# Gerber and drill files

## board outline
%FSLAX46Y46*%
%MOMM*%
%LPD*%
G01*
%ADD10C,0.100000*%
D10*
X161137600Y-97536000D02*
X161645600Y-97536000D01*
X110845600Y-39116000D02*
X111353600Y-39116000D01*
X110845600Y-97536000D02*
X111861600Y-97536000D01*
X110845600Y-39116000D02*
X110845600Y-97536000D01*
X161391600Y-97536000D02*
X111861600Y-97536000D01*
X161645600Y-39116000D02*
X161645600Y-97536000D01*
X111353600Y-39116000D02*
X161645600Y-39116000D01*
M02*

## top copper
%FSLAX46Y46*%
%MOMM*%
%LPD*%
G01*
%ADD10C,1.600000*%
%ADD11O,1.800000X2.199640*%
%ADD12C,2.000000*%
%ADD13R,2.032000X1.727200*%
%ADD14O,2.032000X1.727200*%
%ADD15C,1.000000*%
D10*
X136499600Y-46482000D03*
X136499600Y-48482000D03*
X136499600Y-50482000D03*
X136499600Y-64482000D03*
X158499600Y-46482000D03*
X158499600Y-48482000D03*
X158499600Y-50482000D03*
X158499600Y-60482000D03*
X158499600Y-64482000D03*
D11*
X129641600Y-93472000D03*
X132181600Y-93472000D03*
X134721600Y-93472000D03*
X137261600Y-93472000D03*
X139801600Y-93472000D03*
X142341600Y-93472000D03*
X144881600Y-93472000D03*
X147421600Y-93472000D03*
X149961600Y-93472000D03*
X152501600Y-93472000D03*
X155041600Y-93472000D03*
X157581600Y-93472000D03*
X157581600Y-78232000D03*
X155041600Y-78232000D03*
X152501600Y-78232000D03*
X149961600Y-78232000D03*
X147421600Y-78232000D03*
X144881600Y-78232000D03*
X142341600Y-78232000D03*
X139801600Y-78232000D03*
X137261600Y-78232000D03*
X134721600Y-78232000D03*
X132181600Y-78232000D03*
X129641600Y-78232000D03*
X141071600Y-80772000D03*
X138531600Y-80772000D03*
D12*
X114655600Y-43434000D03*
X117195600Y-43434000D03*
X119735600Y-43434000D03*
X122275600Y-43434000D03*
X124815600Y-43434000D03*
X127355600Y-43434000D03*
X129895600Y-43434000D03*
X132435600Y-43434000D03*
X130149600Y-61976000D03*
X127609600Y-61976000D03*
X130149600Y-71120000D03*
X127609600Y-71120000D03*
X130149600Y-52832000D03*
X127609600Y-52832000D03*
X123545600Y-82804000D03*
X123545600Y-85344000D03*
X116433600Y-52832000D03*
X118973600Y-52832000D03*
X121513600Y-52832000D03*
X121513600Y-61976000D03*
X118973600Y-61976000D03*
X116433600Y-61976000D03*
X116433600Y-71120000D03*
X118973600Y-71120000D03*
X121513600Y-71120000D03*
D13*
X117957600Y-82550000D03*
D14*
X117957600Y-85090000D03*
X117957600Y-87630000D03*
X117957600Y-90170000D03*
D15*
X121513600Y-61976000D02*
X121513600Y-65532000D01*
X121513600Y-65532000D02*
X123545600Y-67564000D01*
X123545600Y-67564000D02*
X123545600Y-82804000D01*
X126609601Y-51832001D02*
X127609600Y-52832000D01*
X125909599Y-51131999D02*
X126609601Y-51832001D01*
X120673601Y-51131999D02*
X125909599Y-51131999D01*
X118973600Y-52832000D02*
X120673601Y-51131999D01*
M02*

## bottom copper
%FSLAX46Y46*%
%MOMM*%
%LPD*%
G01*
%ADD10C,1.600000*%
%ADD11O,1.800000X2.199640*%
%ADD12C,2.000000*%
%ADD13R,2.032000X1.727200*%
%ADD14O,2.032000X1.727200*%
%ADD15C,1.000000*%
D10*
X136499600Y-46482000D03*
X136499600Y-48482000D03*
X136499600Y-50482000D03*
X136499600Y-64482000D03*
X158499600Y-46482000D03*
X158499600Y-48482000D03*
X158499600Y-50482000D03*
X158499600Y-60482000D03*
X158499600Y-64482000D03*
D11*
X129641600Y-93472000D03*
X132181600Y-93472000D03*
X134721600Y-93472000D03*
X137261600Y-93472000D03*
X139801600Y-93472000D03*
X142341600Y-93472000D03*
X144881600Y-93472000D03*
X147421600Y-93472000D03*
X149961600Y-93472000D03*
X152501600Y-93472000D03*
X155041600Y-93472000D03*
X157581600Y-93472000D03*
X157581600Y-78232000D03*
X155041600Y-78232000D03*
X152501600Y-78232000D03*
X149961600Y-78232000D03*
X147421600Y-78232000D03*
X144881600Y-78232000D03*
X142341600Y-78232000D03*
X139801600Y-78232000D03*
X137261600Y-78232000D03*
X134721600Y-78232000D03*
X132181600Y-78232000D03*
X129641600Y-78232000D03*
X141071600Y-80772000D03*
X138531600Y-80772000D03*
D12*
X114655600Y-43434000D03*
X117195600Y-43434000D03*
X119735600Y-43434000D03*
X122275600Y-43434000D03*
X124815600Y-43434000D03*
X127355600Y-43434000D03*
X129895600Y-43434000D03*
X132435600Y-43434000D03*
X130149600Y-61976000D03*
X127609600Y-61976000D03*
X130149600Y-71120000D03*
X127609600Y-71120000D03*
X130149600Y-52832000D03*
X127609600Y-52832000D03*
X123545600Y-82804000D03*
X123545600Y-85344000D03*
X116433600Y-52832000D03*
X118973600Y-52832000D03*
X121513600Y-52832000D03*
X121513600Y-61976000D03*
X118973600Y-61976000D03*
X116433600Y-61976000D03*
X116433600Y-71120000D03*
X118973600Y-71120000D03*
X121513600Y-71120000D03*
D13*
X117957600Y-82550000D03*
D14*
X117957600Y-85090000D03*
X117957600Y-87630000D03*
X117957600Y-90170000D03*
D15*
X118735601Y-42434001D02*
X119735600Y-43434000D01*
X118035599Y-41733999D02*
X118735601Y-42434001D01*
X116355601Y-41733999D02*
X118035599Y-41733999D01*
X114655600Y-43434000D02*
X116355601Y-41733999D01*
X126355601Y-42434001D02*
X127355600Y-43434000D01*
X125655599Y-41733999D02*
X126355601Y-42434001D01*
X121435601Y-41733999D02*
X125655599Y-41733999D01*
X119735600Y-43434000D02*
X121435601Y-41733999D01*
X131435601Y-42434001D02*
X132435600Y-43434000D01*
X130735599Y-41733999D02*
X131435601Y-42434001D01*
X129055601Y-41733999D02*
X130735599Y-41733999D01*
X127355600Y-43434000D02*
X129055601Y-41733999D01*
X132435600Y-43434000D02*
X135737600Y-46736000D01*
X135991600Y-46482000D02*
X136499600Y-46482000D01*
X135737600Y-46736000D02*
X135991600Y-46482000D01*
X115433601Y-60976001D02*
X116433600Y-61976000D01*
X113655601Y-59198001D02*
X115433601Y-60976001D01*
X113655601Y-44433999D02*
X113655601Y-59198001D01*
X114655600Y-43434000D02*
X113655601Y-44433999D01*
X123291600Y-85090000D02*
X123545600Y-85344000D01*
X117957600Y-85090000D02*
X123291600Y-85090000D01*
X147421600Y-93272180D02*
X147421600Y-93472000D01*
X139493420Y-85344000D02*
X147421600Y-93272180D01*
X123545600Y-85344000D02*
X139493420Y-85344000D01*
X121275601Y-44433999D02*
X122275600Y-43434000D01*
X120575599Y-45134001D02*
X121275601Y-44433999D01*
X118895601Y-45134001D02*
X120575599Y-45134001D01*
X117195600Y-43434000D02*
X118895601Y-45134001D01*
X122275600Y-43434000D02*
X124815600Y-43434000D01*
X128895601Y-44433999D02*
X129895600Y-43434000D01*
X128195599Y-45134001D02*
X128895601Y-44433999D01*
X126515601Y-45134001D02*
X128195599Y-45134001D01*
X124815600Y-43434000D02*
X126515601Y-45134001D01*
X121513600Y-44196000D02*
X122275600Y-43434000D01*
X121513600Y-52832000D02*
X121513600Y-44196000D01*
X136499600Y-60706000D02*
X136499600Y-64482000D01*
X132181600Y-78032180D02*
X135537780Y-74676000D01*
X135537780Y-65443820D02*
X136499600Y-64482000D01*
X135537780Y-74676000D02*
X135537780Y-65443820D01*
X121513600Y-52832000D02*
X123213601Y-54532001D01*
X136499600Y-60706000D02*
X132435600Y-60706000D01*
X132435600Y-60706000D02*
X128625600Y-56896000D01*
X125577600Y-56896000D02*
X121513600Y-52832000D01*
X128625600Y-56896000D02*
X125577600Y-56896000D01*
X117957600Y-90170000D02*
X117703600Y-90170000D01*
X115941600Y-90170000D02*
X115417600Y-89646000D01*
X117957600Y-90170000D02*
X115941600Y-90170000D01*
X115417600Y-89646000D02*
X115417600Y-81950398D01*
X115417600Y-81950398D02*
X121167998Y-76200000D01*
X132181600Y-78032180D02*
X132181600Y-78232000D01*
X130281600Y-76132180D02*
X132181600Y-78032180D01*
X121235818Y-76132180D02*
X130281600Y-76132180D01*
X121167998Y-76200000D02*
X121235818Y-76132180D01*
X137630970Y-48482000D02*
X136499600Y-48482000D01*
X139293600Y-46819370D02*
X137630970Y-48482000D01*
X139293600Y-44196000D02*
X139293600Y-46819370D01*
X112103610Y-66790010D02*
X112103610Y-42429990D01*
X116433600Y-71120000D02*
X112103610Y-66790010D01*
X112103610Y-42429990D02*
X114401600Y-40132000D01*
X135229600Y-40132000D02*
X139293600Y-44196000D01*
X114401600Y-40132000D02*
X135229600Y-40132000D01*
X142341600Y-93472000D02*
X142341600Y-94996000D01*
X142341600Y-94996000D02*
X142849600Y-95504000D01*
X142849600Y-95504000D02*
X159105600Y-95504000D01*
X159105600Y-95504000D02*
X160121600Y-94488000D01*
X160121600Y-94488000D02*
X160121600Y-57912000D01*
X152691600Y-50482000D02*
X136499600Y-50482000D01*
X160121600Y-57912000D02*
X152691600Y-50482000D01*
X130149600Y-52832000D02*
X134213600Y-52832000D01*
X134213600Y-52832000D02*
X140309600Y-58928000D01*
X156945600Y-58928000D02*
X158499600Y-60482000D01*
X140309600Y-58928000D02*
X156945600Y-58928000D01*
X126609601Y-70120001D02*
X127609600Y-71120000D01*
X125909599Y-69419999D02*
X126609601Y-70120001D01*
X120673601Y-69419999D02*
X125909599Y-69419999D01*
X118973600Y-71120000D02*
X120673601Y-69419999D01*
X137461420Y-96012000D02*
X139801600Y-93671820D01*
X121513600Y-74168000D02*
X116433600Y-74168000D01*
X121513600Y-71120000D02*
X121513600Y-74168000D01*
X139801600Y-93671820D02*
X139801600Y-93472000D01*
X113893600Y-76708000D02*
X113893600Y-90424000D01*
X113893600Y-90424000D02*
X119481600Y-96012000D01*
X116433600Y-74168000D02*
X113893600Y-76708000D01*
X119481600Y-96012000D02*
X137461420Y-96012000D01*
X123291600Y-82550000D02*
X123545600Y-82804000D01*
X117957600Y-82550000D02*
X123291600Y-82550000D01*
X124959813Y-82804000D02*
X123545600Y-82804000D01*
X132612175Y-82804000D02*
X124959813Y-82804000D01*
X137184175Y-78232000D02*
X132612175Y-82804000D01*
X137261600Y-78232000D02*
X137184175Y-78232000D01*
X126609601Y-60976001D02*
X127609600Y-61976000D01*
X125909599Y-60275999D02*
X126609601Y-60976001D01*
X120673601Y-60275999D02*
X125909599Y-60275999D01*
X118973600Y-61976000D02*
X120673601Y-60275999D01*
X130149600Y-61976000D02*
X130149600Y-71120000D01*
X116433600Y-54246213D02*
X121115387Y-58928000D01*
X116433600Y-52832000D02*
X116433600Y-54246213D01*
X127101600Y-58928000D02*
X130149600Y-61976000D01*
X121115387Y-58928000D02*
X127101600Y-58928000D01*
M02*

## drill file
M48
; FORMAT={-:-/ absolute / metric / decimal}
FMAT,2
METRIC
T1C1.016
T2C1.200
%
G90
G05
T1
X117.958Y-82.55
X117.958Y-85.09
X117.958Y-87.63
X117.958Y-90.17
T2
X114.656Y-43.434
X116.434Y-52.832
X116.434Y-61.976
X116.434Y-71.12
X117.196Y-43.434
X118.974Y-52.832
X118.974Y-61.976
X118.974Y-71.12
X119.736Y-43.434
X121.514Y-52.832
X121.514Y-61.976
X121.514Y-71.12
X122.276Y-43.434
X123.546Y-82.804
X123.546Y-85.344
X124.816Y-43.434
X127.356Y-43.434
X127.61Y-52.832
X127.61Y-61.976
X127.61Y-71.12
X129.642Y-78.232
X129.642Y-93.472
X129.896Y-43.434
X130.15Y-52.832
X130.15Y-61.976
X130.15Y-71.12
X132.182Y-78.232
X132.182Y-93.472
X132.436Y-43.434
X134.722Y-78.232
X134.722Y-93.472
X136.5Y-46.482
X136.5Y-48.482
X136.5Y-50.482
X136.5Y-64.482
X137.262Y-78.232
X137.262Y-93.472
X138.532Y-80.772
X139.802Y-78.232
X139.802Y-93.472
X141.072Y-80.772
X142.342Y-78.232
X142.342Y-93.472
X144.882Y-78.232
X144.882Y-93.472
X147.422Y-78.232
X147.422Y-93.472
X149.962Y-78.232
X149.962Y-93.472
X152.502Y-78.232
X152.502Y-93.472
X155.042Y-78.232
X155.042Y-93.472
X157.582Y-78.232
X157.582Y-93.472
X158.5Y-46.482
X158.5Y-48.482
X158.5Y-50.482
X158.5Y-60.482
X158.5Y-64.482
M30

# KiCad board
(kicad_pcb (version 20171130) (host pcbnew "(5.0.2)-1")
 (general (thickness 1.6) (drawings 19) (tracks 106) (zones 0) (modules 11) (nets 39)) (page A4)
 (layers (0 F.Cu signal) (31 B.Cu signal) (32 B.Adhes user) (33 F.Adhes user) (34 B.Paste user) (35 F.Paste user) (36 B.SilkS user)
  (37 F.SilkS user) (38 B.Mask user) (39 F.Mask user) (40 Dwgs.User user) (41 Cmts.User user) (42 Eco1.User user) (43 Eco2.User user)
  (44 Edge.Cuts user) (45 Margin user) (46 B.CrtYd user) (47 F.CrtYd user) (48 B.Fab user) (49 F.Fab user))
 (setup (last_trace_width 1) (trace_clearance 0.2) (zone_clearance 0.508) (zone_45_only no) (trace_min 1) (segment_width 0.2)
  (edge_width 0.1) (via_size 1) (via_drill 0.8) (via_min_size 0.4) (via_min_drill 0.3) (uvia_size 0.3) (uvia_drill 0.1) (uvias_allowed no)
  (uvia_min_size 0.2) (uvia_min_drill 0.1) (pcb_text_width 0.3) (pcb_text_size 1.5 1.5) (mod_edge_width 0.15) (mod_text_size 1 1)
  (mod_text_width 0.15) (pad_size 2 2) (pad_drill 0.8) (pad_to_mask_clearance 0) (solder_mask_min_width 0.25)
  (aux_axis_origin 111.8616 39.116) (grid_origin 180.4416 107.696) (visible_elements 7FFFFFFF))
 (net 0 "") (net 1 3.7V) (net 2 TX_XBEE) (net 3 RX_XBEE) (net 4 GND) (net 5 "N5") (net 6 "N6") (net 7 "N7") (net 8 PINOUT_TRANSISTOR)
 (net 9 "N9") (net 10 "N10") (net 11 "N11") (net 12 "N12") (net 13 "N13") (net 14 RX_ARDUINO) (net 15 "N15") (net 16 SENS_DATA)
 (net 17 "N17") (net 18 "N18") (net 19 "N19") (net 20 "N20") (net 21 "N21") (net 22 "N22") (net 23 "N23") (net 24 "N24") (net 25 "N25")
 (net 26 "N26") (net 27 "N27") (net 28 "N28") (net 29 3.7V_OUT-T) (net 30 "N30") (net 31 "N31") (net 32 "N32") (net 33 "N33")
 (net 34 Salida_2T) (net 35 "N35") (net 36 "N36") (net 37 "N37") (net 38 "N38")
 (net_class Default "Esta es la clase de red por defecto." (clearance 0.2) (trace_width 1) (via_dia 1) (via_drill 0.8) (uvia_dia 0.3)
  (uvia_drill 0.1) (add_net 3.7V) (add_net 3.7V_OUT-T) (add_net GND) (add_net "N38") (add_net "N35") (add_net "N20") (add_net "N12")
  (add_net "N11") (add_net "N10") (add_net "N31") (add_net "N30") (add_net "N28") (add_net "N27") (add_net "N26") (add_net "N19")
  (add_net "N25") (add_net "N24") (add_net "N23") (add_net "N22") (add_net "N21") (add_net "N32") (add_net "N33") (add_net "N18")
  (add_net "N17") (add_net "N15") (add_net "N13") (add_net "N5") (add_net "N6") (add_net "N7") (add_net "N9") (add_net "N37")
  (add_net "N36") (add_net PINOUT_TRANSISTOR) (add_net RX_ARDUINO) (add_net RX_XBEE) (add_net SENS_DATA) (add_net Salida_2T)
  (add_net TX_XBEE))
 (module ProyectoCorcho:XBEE (layer F.Cu) (at 135.2296 45.212)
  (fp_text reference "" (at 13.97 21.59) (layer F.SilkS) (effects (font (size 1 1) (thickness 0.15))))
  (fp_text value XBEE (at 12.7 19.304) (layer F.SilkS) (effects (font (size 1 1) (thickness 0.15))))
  (pad 1 thru_hole circle (at 1.27 1.27) (size 1.6 1.6) (drill 1.2) (layers *.Cu *.Mask) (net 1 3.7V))
  (pad 2 thru_hole circle (at 1.27 3.27) (size 1.6 1.6) (drill 1.2) (layers *.Cu *.Mask) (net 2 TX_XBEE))
  (pad 3 thru_hole circle (at 1.27 5.27) (size 1.6 1.6) (drill 1.2) (layers *.Cu *.Mask) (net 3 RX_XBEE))
  (pad 4 thru_hole circle (at 1.27 19.27) (size 1.6 1.6) (drill 1.2) (layers *.Cu *.Mask) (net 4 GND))
  (pad 5 thru_hole circle (at 23.27 1.27) (size 1.6 1.6) (drill 1.2) (layers *.Cu *.Mask) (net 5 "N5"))
  (pad 6 thru_hole circle (at 23.27 3.27) (size 1.6 1.6) (drill 1.2) (layers *.Cu *.Mask) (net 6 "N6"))
  (pad 7 thru_hole circle (at 23.27 5.27) (size 1.6 1.6) (drill 1.2) (layers *.Cu *.Mask) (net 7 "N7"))
  (pad 8 thru_hole circle (at 23.27 15.27) (size 1.6 1.6) (drill 1.2) (layers *.Cu *.Mask) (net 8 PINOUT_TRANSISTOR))
  (pad 9 thru_hole circle (at 23.27 19.27) (size 1.6 1.6) (drill 1.2) (layers *.Cu *.Mask) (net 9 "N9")))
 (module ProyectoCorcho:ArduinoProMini (layer F.Cu) (at 143.6116 85.852)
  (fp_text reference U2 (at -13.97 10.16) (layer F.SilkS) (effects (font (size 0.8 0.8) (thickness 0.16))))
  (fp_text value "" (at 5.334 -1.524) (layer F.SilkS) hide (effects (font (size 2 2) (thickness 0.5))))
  (pad 12 thru_hole oval (at -13.97 7.62) (size 1.8 2.19964) (drill 1.2) (layers *.Cu *.Mask) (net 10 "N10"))
  (pad 11 thru_hole oval (at -11.43 7.62) (size 1.8 2.19964) (drill 1.2) (layers *.Cu *.Mask) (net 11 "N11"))
  (pad 10 thru_hole oval (at -8.89 7.62) (size 1.8 2.19964) (drill 1.2) (layers *.Cu *.Mask) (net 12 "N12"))
  (pad 9 thru_hole oval (at -6.35 7.62) (size 1.8 2.19964) (drill 1.2) (layers *.Cu *.Mask) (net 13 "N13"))
  (pad 8 thru_hole oval (at -3.81 7.62) (size 1.8 2.19964) (drill 1.2) (layers *.Cu *.Mask) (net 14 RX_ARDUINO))
  (pad 7 thru_hole oval (at -1.27 7.62) (size 1.8 2.19964) (drill 1.2) (layers *.Cu *.Mask) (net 3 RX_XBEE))
  (pad 6 thru_hole oval (at 1.27 7.62) (size 1.8 2.19964) (drill 1.2) (layers *.Cu *.Mask) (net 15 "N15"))
  (pad 5 thru_hole oval (at 3.81 7.62) (size 1.8 2.19964) (drill 1.2) (layers *.Cu *.Mask) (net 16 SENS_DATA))
  (pad 4 thru_hole oval (at 6.35 7.62) (size 1.8 2.19964) (drill 1.2) (layers *.Cu *.Mask) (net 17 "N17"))
  (pad 3 thru_hole oval (at 8.89 7.62) (size 1.8 2.19964) (drill 1.2) (layers *.Cu *.Mask) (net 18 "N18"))
  (pad 2 thru_hole oval (at 11.43 7.62) (size 1.8 2.19964) (drill 1.2) (layers *.Cu *.Mask) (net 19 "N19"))
  (pad 1 thru_hole oval (at 13.97 7.62) (size 1.8 2.19964) (drill 1.2) (layers *.Cu *.Mask) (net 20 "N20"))
  (pad 24 thru_hole oval (at 13.97 -7.62) (size 1.8 2.19964) (drill 1.2) (layers *.Cu *.Mask) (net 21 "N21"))
  (pad 23 thru_hole oval (at 11.43 -7.62) (size 1.8 2.19964) (drill 1.2) (layers *.Cu *.Mask) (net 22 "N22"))
  (pad 22 thru_hole oval (at 8.89 -7.62) (size 1.8 2.19964) (drill 1.2) (layers *.Cu *.Mask) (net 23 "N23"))
  (pad 21 thru_hole oval (at 6.35 -7.62) (size 1.8 2.19964) (drill 1.2) (layers *.Cu *.Mask) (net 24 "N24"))
  (pad 20 thru_hole oval (at 3.81 -7.62) (size 1.8 2.19964) (drill 1.2) (layers *.Cu *.Mask) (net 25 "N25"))
  (pad 19 thru_hole oval (at 1.27 -7.62) (size 1.8 2.19964) (drill 1.2) (layers *.Cu *.Mask) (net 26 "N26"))
  (pad 18 thru_hole oval (at -1.27 -7.62) (size 1.8 2.19964) (drill 1.2) (layers *.Cu *.Mask) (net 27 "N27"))
  (pad 17 thru_hole oval (at -3.81 -7.62) (size 1.8 2.19964) (drill 1.2) (layers *.Cu *.Mask) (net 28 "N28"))
  (pad 16 thru_hole oval (at -6.35 -7.62) (size 1.8 2.19964) (drill 1.2) (layers *.Cu *.Mask) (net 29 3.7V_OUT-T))
  (pad 15 thru_hole oval (at -8.89 -7.62) (size 1.8 2.19964) (drill 1.2) (layers *.Cu *.Mask) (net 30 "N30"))
  (pad 14 thru_hole oval (at -11.43 -7.62) (size 1.8 2.19964) (drill 1.2) (layers *.Cu *.Mask) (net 4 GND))
  (pad 13 thru_hole oval (at -13.97 -7.62) (size 1.8 2.19964) (drill 1.2) (layers *.Cu *.Mask) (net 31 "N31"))
  (pad 25 thru_hole oval (at -2.54 -5.08) (size 1.8 2.19964) (drill 1.2) (layers *.Cu *.Mask) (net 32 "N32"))
  (pad 26 thru_hole oval (at -5.08 -5.08) (size 1.8 2.19964) (drill 1.2) (layers *.Cu *.Mask) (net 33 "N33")))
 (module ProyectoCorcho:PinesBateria (layer F.Cu) (at 113.3856 42.164)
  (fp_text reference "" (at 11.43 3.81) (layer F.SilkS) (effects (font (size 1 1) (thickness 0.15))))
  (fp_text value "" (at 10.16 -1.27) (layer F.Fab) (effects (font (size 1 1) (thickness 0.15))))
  (pad 1 thru_hole circle (at 1.27 1.27) (size 2 2) (drill 1.2) (layers *.Cu *.Mask) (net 1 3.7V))
  (pad 2 thru_hole circle (at 3.81 1.27) (size 2 2) (drill 1.2) (layers *.Cu *.Mask) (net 4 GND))
  (pad 3 thru_hole circle (at 6.35 1.27) (size 2 2) (drill 1.2) (layers *.Cu *.Mask) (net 1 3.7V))
  (pad 4 thru_hole circle (at 8.89 1.27) (size 2 2) (drill 1.2) (layers *.Cu *.Mask) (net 4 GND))
  (pad 5 thru_hole circle (at 11.43 1.27) (size 2 2) (drill 1.2) (layers *.Cu *.Mask) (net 4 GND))
  (pad 6 thru_hole circle (at 13.97 1.27) (size 2 2) (drill 1.2) (layers *.Cu *.Mask) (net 1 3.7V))
  (pad 7 thru_hole circle (at 16.51 1.27) (size 2 2) (drill 1.2) (layers *.Cu *.Mask) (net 4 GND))
  (pad 8 thru_hole circle (at 19.05 1.27) (size 2 2) (drill 1.2) (layers *.Cu *.Mask) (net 1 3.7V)))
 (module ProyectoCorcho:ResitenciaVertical (layer F.Cu) (at 127.6096 61.976)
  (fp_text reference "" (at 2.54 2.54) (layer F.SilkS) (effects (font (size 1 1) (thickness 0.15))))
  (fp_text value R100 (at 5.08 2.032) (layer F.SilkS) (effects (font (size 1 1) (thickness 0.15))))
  (pad 2 thru_hole circle (at 2.54 0) (size 2 2) (drill 1.2) (layers *.Cu *.Mask) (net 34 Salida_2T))
  (pad 1 thru_hole circle (at 0 0) (size 2 2) (drill 1.2) (layers *.Cu *.Mask) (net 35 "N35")))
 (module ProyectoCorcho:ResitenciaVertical (layer F.Cu) (at 127.6096 71.12)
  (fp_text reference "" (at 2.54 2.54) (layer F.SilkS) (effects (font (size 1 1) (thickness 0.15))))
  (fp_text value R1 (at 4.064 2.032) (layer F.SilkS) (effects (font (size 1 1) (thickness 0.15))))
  (pad 2 thru_hole circle (at 2.54 0) (size 2 2) (drill 1.2) (layers *.Cu *.Mask) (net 34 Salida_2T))
  (pad 1 thru_hole circle (at 0 0) (size 2 2) (drill 1.2) (layers *.Cu *.Mask) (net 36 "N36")))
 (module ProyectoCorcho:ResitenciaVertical (layer F.Cu) (at 127.6096 52.832)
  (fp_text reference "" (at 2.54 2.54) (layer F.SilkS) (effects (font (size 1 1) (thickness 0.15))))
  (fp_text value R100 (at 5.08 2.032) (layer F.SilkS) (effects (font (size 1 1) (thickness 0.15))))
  (pad 2 thru_hole circle (at 2.54 0) (size 2 2) (drill 1.2) (layers *.Cu *.Mask) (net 8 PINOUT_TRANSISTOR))
  (pad 1 thru_hole circle (at 0 0) (size 2 2) (drill 1.2) (layers *.Cu *.Mask) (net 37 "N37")))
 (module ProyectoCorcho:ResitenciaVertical (layer F.Cu) (at 123.5456 82.804 270)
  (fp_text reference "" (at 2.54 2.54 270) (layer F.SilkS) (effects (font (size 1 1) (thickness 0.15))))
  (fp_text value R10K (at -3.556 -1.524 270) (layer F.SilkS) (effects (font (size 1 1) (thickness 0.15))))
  (pad 1 thru_hole circle (at 0 0 270) (size 2 2) (drill 1.2) (layers *.Cu *.Mask) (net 29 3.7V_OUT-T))
  (pad 2 thru_hole circle (at 2.54 0 270) (size 2 2) (drill 1.2) (layers *.Cu *.Mask) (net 16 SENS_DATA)))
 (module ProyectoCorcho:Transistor (layer F.Cu) (at 118.9736 52.832)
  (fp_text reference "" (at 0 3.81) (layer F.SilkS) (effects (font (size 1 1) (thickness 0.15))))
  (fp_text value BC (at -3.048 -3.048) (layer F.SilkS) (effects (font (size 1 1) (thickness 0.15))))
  (pad 1 thru_hole circle (at -2.54 0) (size 2 2) (drill 1.2) (layers *.Cu *.Mask) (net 34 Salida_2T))
  (pad 2 thru_hole circle (at 0 0) (size 2 2) (drill 1.2) (layers *.Cu *.Mask) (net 37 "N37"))
  (pad 3 thru_hole circle (at 2.54 0) (size 2 2) (drill 1.2) (layers *.Cu *.Mask) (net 4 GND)))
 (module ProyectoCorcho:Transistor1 (layer B.Cu) (at 118.9736 61.976)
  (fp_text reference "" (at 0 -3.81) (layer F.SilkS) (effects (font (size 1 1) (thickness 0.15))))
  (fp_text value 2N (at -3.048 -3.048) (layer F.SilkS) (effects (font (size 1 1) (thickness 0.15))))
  (pad 3 thru_hole circle (at 2.54 0) (size 2 2) (drill 1.2) (layers *.Cu *.Mask) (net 29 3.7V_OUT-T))
  (pad 2 thru_hole circle (at 0 0) (size 2 2) (drill 1.2) (layers *.Cu *.Mask) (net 35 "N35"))
  (pad 1 thru_hole circle (at -2.54 0) (size 2 2) (drill 1.2) (layers *.Cu *.Mask) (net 1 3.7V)))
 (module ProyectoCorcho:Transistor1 (layer F.Cu) (at 118.9736 71.12)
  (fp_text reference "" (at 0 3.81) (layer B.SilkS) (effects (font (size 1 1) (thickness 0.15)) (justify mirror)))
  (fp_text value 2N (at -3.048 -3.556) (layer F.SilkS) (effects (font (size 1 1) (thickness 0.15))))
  (pad 1 thru_hole circle (at -2.54 0) (size 2 2) (drill 1.2) (layers *.Cu *.Mask) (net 2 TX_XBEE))
  (pad 2 thru_hole circle (at 0 0) (size 2 2) (drill 1.2) (layers *.Cu *.Mask) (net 36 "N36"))
  (pad 3 thru_hole circle (at 2.54 0) (size 2 2) (drill 1.2) (layers *.Cu *.Mask) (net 14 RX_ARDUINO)))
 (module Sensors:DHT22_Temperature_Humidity (layer F.Cu) (at 117.9576 86.36 270)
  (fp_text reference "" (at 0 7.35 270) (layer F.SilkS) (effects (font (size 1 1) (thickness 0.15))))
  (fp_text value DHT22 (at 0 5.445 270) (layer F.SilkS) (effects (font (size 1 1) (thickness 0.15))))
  (pad 1 thru_hole rect (at -3.81 0) (size 2.032 1.7272) (drill 1.016) (layers *.Cu *.Mask F.SilkS) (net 29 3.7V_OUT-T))
  (pad 2 thru_hole oval (at -1.27 0) (size 2.032 1.7272) (drill 1.016) (layers *.Cu *.Mask F.SilkS) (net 16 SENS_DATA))
  (pad 3 thru_hole oval (at 1.27 0) (size 2.032 1.7272) (drill 1.016) (layers *.Cu *.Mask F.SilkS) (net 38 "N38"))
  (pad 4 thru_hole oval (at 3.81 0) (size 2.032 1.7272) (drill 1.016) (layers *.Cu *.Mask F.SilkS) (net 4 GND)))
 (gr_line (start 161.1376 97.536) (end 161.6456 97.536) (layer Edge.Cuts) (width 0.1))
 (gr_line (start 110.8456 39.116) (end 111.3536 39.116) (layer Edge.Cuts) (width 0.1))
 (gr_line (start 110.8456 97.536) (end 111.8616 97.536) (layer Edge.Cuts) (width 0.1))
 (gr_line (start 110.8456 39.116) (end 110.8456 97.536) (layer Edge.Cuts) (width 0.1))
 (gr_line (start 161.3916 97.536) (end 111.8616 97.536) (layer Edge.Cuts) (width 0.1))
 (gr_line (start 161.6456 39.116) (end 161.6456 97.536) (layer Edge.Cuts) (width 0.1))
 (gr_line (start 111.3536 39.116) (end 161.6456 39.116) (layer Edge.Cuts) (width 0.1))
 (segment (start 118.735601 42.434001) (end 119.7356 43.434) (width 1) (layer B.Cu) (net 1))
 (segment (start 118.035599 41.733999) (end 118.735601 42.434001) (width 1) (layer B.Cu) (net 1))
 (segment (start 116.355601 41.733999) (end 118.035599 41.733999) (width 1) (layer B.Cu) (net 1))
 (segment (start 114.6556 43.434) (end 116.355601 41.733999) (width 1) (layer B.Cu) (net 1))
 (segment (start 126.355601 42.434001) (end 127.3556 43.434) (width 1) (layer B.Cu) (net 1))
 (segment (start 125.655599 41.733999) (end 126.355601 42.434001) (width 1) (layer B.Cu) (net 1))
 (segment (start 121.435601 41.733999) (end 125.655599 41.733999) (width 1) (layer B.Cu) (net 1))
 (segment (start 119.7356 43.434) (end 121.435601 41.733999) (width 1) (layer B.Cu) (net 1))
 (segment (start 131.435601 42.434001) (end 132.4356 43.434) (width 1) (layer B.Cu) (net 1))
 (segment (start 130.735599 41.733999) (end 131.435601 42.434001) (width 1) (layer B.Cu) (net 1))
 (segment (start 129.055601 41.733999) (end 130.735599 41.733999) (width 1) (layer B.Cu) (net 1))
 (segment (start 127.3556 43.434) (end 129.055601 41.733999) (width 1) (layer B.Cu) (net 1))
 (segment (start 132.4356 43.434) (end 135.7376 46.736) (width 1) (layer B.Cu) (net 1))
 (segment (start 135.9916 46.482) (end 136.4996 46.482) (width 1) (layer B.Cu) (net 1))
 (segment (start 135.7376 46.736) (end 135.9916 46.482) (width 1) (layer B.Cu) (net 1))
 (segment (start 115.433601 60.976001) (end 116.4336 61.976) (width 1) (layer B.Cu) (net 1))
 (segment (start 113.655601 59.198001) (end 115.433601 60.976001) (width 1) (layer B.Cu) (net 1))
 (segment (start 113.655601 44.433999) (end 113.655601 59.198001) (width 1) (layer B.Cu) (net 1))
 (segment (start 114.6556 43.434) (end 113.655601 44.433999) (width 1) (layer B.Cu) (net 1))
 (segment (start 123.2916 85.09) (end 123.5456 85.344) (width 1) (layer B.Cu) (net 16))
 (segment (start 117.9576 85.09) (end 123.2916 85.09) (width 1) (layer B.Cu) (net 16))
 (segment (start 147.4216 93.27218) (end 147.4216 93.472) (width 1) (layer B.Cu) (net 16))
 (segment (start 139.49342 85.344) (end 147.4216 93.27218) (width 1) (layer B.Cu) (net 16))
 (segment (start 123.5456 85.344) (end 139.49342 85.344) (width 1) (layer B.Cu) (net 16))
 (segment (start 121.275601 44.433999) (end 122.2756 43.434) (width 1) (layer B.Cu) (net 4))
 (segment (start 120.575599 45.134001) (end 121.275601 44.433999) (width 1) (layer B.Cu) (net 4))
 (segment (start 118.895601 45.134001) (end 120.575599 45.134001) (width 1) (layer B.Cu) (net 4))
 (segment (start 117.1956 43.434) (end 118.895601 45.134001) (width 1) (layer B.Cu) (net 4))
 (segment (start 122.2756 43.434) (end 124.8156 43.434) (width 1) (layer B.Cu) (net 4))
 (segment (start 128.895601 44.433999) (end 129.8956 43.434) (width 1) (layer B.Cu) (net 4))
 (segment (start 128.195599 45.134001) (end 128.895601 44.433999) (width 1) (layer B.Cu) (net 4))
 (segment (start 126.515601 45.134001) (end 128.195599 45.134001) (width 1) (layer B.Cu) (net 4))
 (segment (start 124.8156 43.434) (end 126.515601 45.134001) (width 1) (layer B.Cu) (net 4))
 (segment (start 121.5136 44.196) (end 122.2756 43.434) (width 1) (layer B.Cu) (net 4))
 (segment (start 121.5136 52.832) (end 121.5136 44.196) (width 1) (layer B.Cu) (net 4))
 (segment (start 136.4996 60.706) (end 136.4996 64.482) (width 1) (layer B.Cu) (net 4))
 (segment (start 132.1816 78.03218) (end 135.53778 74.676) (width 1) (layer B.Cu) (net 4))
 (segment (start 135.53778 65.44382) (end 136.4996 64.482) (width 1) (layer B.Cu) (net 4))
 (segment (start 135.53778 74.676) (end 135.53778 65.44382) (width 1) (layer B.Cu) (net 4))
 (segment (start 121.5136 52.832) (end 123.213601 54.532001) (width 1) (layer B.Cu) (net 4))
 (segment (start 136.4996 60.706) (end 132.4356 60.706) (width 1) (layer B.Cu) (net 4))
 (segment (start 132.4356 60.706) (end 128.6256 56.896) (width 1) (layer B.Cu) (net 4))
 (segment (start 125.5776 56.896) (end 121.5136 52.832) (width 1) (layer B.Cu) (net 4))
 (segment (start 128.6256 56.896) (end 125.5776 56.896) (width 1) (layer B.Cu) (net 4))
 (segment (start 117.9576 90.17) (end 117.7036 90.17) (width 1) (layer B.Cu) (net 4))
 (segment (start 115.9416 90.17) (end 115.4176 89.646) (width 1) (layer B.Cu) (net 4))
 (segment (start 117.9576 90.17) (end 115.9416 90.17) (width 1) (layer B.Cu) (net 4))
 (segment (start 115.4176 89.646) (end 115.4176 81.950398) (width 1) (layer B.Cu) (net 4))
 (segment (start 115.4176 81.950398) (end 121.167998 76.2) (width 1) (layer B.Cu) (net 4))
 (segment (start 132.1816 78.03218) (end 132.1816 78.232) (width 1) (layer B.Cu) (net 4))
 (segment (start 130.2816 76.13218) (end 132.1816 78.03218) (width 1) (layer B.Cu) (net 4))
 (segment (start 121.235818 76.13218) (end 130.2816 76.13218) (width 1) (layer B.Cu) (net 4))
 (segment (start 121.167998 76.2) (end 121.235818 76.13218) (width 1) (layer B.Cu) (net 4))
 (segment (start 137.63097 48.482) (end 136.4996 48.482) (width 1) (layer B.Cu) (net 2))
 (segment (start 139.2936 46.81937) (end 137.63097 48.482) (width 1) (layer B.Cu) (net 2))
 (segment (start 139.2936 44.196) (end 139.2936 46.81937) (width 1) (layer B.Cu) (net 2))
 (segment (start 112.10361 66.79001) (end 112.10361 42.42999) (width 1) (layer B.Cu) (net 2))
 (segment (start 116.4336 71.12) (end 112.10361 66.79001) (width 1) (layer B.Cu) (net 2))
 (segment (start 112.10361 42.42999) (end 114.4016 40.132) (width 1) (layer B.Cu) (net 2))
 (segment (start 135.2296 40.132) (end 139.2936 44.196) (width 1) (layer B.Cu) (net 2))
 (segment (start 114.4016 40.132) (end 135.2296 40.132) (width 1) (layer B.Cu) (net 2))
 (segment (start 142.3416 93.472) (end 142.3416 94.996) (width 1) (layer B.Cu) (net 3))
 (segment (start 142.3416 94.996) (end 142.8496 95.504) (width 1) (layer B.Cu) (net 3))
 (segment (start 142.8496 95.504) (end 159.1056 95.504) (width 1) (layer B.Cu) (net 3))
 (segment (start 159.1056 95.504) (end 160.1216 94.488) (width 1) (layer B.Cu) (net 3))
 (segment (start 160.1216 94.488) (end 160.1216 57.912) (width 1) (layer B.Cu) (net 3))
 (segment (start 152.6916 50.482) (end 136.4996 50.482) (width 1) (layer B.Cu) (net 3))
 (segment (start 160.1216 57.912) (end 152.6916 50.482) (width 1) (layer B.Cu) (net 3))
 (segment (start 130.1496 52.832) (end 134.2136 52.832) (width 1) (layer B.Cu) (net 8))
 (segment (start 134.2136 52.832) (end 140.3096 58.928) (width 1) (layer B.Cu) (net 8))
 (segment (start 156.9456 58.928) (end 158.4996 60.482) (width 1) (layer B.Cu) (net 8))
 (segment (start 140.3096 58.928) (end 156.9456 58.928) (width 1) (layer B.Cu) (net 8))
 (segment (start 126.609601 70.120001) (end 127.6096 71.12) (width 1) (layer B.Cu) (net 36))
 (segment (start 125.909599 69.419999) (end 126.609601 70.120001) (width 1) (layer B.Cu) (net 36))
 (segment (start 120.673601 69.419999) (end 125.909599 69.419999) (width 1) (layer B.Cu) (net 36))
 (segment (start 118.9736 71.12) (end 120.673601 69.419999) (width 1) (layer B.Cu) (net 36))
 (segment (start 137.46142 96.012) (end 139.8016 93.67182) (width 1) (layer B.Cu) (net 14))
 (segment (start 121.5136 74.168) (end 116.4336 74.168) (width 1) (layer B.Cu) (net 14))
 (segment (start 121.5136 71.12) (end 121.5136 74.168) (width 1) (layer B.Cu) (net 14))
 (segment (start 139.8016 93.67182) (end 139.8016 93.472) (width 1) (layer B.Cu) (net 14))
 (segment (start 113.8936 76.708) (end 113.8936 90.424) (width 1) (layer B.Cu) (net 14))
 (segment (start 113.8936 90.424) (end 119.4816 96.012) (width 1) (layer B.Cu) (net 14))
 (segment (start 116.4336 74.168) (end 113.8936 76.708) (width 1) (layer B.Cu) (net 14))
 (segment (start 119.4816 96.012) (end 137.46142 96.012) (width 1) (layer B.Cu) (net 14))
 (segment (start 123.2916 82.55) (end 123.5456 82.804) (width 1) (layer B.Cu) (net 29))
 (segment (start 117.9576 82.55) (end 123.2916 82.55) (width 1) (layer B.Cu) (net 29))
 (segment (start 124.959813 82.804) (end 123.5456 82.804) (width 1) (layer B.Cu) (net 29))
 (segment (start 132.612175 82.804) (end 124.959813 82.804) (width 1) (layer B.Cu) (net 29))
 (segment (start 137.184175 78.232) (end 132.612175 82.804) (width 1) (layer B.Cu) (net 29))
 (segment (start 137.2616 78.232) (end 137.184175 78.232) (width 1) (layer B.Cu) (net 29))
 (segment (start 121.5136 61.976) (end 121.5136 65.532) (width 1) (layer F.Cu) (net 29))
 (segment (start 121.5136 65.532) (end 123.5456 67.564) (width 1) (layer F.Cu) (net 29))
 (segment (start 123.5456 67.564) (end 123.5456 82.804) (width 1) (layer F.Cu) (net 29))
 (segment (start 126.609601 60.976001) (end 127.6096 61.976) (width 1) (layer B.Cu) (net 35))
 (segment (start 125.909599 60.275999) (end 126.609601 60.976001) (width 1) (layer B.Cu) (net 35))
 (segment (start 120.673601 60.275999) (end 125.909599 60.275999) (width 1) (layer B.Cu) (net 35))
 (segment (start 118.9736 61.976) (end 120.673601 60.275999) (width 1) (layer B.Cu) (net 35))
 (segment (start 130.1496 61.976) (end 130.1496 71.12) (width 1) (layer B.Cu) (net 34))
 (segment (start 116.4336 54.246213) (end 121.115387 58.928) (width 1) (layer B.Cu) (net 34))
 (segment (start 116.4336 52.832) (end 116.4336 54.246213) (width 1) (layer B.Cu) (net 34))
 (segment (start 127.1016 58.928) (end 130.1496 61.976) (width 1) (layer B.Cu) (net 34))
 (segment (start 121.115387 58.928) (end 127.1016 58.928) (width 1) (layer B.Cu) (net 34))
 (segment (start 126.609601 51.832001) (end 127.6096 52.832) (width 1) (layer F.Cu) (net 37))
 (segment (start 125.909599 51.131999) (end 126.609601 51.832001) (width 1) (layer F.Cu) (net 37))
 (segment (start 120.673601 51.131999) (end 125.909599 51.131999) (width 1) (layer F.Cu) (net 37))
 (segment (start 118.9736 52.832) (end 120.673601 51.131999) (width 1) (layer F.Cu) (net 37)))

